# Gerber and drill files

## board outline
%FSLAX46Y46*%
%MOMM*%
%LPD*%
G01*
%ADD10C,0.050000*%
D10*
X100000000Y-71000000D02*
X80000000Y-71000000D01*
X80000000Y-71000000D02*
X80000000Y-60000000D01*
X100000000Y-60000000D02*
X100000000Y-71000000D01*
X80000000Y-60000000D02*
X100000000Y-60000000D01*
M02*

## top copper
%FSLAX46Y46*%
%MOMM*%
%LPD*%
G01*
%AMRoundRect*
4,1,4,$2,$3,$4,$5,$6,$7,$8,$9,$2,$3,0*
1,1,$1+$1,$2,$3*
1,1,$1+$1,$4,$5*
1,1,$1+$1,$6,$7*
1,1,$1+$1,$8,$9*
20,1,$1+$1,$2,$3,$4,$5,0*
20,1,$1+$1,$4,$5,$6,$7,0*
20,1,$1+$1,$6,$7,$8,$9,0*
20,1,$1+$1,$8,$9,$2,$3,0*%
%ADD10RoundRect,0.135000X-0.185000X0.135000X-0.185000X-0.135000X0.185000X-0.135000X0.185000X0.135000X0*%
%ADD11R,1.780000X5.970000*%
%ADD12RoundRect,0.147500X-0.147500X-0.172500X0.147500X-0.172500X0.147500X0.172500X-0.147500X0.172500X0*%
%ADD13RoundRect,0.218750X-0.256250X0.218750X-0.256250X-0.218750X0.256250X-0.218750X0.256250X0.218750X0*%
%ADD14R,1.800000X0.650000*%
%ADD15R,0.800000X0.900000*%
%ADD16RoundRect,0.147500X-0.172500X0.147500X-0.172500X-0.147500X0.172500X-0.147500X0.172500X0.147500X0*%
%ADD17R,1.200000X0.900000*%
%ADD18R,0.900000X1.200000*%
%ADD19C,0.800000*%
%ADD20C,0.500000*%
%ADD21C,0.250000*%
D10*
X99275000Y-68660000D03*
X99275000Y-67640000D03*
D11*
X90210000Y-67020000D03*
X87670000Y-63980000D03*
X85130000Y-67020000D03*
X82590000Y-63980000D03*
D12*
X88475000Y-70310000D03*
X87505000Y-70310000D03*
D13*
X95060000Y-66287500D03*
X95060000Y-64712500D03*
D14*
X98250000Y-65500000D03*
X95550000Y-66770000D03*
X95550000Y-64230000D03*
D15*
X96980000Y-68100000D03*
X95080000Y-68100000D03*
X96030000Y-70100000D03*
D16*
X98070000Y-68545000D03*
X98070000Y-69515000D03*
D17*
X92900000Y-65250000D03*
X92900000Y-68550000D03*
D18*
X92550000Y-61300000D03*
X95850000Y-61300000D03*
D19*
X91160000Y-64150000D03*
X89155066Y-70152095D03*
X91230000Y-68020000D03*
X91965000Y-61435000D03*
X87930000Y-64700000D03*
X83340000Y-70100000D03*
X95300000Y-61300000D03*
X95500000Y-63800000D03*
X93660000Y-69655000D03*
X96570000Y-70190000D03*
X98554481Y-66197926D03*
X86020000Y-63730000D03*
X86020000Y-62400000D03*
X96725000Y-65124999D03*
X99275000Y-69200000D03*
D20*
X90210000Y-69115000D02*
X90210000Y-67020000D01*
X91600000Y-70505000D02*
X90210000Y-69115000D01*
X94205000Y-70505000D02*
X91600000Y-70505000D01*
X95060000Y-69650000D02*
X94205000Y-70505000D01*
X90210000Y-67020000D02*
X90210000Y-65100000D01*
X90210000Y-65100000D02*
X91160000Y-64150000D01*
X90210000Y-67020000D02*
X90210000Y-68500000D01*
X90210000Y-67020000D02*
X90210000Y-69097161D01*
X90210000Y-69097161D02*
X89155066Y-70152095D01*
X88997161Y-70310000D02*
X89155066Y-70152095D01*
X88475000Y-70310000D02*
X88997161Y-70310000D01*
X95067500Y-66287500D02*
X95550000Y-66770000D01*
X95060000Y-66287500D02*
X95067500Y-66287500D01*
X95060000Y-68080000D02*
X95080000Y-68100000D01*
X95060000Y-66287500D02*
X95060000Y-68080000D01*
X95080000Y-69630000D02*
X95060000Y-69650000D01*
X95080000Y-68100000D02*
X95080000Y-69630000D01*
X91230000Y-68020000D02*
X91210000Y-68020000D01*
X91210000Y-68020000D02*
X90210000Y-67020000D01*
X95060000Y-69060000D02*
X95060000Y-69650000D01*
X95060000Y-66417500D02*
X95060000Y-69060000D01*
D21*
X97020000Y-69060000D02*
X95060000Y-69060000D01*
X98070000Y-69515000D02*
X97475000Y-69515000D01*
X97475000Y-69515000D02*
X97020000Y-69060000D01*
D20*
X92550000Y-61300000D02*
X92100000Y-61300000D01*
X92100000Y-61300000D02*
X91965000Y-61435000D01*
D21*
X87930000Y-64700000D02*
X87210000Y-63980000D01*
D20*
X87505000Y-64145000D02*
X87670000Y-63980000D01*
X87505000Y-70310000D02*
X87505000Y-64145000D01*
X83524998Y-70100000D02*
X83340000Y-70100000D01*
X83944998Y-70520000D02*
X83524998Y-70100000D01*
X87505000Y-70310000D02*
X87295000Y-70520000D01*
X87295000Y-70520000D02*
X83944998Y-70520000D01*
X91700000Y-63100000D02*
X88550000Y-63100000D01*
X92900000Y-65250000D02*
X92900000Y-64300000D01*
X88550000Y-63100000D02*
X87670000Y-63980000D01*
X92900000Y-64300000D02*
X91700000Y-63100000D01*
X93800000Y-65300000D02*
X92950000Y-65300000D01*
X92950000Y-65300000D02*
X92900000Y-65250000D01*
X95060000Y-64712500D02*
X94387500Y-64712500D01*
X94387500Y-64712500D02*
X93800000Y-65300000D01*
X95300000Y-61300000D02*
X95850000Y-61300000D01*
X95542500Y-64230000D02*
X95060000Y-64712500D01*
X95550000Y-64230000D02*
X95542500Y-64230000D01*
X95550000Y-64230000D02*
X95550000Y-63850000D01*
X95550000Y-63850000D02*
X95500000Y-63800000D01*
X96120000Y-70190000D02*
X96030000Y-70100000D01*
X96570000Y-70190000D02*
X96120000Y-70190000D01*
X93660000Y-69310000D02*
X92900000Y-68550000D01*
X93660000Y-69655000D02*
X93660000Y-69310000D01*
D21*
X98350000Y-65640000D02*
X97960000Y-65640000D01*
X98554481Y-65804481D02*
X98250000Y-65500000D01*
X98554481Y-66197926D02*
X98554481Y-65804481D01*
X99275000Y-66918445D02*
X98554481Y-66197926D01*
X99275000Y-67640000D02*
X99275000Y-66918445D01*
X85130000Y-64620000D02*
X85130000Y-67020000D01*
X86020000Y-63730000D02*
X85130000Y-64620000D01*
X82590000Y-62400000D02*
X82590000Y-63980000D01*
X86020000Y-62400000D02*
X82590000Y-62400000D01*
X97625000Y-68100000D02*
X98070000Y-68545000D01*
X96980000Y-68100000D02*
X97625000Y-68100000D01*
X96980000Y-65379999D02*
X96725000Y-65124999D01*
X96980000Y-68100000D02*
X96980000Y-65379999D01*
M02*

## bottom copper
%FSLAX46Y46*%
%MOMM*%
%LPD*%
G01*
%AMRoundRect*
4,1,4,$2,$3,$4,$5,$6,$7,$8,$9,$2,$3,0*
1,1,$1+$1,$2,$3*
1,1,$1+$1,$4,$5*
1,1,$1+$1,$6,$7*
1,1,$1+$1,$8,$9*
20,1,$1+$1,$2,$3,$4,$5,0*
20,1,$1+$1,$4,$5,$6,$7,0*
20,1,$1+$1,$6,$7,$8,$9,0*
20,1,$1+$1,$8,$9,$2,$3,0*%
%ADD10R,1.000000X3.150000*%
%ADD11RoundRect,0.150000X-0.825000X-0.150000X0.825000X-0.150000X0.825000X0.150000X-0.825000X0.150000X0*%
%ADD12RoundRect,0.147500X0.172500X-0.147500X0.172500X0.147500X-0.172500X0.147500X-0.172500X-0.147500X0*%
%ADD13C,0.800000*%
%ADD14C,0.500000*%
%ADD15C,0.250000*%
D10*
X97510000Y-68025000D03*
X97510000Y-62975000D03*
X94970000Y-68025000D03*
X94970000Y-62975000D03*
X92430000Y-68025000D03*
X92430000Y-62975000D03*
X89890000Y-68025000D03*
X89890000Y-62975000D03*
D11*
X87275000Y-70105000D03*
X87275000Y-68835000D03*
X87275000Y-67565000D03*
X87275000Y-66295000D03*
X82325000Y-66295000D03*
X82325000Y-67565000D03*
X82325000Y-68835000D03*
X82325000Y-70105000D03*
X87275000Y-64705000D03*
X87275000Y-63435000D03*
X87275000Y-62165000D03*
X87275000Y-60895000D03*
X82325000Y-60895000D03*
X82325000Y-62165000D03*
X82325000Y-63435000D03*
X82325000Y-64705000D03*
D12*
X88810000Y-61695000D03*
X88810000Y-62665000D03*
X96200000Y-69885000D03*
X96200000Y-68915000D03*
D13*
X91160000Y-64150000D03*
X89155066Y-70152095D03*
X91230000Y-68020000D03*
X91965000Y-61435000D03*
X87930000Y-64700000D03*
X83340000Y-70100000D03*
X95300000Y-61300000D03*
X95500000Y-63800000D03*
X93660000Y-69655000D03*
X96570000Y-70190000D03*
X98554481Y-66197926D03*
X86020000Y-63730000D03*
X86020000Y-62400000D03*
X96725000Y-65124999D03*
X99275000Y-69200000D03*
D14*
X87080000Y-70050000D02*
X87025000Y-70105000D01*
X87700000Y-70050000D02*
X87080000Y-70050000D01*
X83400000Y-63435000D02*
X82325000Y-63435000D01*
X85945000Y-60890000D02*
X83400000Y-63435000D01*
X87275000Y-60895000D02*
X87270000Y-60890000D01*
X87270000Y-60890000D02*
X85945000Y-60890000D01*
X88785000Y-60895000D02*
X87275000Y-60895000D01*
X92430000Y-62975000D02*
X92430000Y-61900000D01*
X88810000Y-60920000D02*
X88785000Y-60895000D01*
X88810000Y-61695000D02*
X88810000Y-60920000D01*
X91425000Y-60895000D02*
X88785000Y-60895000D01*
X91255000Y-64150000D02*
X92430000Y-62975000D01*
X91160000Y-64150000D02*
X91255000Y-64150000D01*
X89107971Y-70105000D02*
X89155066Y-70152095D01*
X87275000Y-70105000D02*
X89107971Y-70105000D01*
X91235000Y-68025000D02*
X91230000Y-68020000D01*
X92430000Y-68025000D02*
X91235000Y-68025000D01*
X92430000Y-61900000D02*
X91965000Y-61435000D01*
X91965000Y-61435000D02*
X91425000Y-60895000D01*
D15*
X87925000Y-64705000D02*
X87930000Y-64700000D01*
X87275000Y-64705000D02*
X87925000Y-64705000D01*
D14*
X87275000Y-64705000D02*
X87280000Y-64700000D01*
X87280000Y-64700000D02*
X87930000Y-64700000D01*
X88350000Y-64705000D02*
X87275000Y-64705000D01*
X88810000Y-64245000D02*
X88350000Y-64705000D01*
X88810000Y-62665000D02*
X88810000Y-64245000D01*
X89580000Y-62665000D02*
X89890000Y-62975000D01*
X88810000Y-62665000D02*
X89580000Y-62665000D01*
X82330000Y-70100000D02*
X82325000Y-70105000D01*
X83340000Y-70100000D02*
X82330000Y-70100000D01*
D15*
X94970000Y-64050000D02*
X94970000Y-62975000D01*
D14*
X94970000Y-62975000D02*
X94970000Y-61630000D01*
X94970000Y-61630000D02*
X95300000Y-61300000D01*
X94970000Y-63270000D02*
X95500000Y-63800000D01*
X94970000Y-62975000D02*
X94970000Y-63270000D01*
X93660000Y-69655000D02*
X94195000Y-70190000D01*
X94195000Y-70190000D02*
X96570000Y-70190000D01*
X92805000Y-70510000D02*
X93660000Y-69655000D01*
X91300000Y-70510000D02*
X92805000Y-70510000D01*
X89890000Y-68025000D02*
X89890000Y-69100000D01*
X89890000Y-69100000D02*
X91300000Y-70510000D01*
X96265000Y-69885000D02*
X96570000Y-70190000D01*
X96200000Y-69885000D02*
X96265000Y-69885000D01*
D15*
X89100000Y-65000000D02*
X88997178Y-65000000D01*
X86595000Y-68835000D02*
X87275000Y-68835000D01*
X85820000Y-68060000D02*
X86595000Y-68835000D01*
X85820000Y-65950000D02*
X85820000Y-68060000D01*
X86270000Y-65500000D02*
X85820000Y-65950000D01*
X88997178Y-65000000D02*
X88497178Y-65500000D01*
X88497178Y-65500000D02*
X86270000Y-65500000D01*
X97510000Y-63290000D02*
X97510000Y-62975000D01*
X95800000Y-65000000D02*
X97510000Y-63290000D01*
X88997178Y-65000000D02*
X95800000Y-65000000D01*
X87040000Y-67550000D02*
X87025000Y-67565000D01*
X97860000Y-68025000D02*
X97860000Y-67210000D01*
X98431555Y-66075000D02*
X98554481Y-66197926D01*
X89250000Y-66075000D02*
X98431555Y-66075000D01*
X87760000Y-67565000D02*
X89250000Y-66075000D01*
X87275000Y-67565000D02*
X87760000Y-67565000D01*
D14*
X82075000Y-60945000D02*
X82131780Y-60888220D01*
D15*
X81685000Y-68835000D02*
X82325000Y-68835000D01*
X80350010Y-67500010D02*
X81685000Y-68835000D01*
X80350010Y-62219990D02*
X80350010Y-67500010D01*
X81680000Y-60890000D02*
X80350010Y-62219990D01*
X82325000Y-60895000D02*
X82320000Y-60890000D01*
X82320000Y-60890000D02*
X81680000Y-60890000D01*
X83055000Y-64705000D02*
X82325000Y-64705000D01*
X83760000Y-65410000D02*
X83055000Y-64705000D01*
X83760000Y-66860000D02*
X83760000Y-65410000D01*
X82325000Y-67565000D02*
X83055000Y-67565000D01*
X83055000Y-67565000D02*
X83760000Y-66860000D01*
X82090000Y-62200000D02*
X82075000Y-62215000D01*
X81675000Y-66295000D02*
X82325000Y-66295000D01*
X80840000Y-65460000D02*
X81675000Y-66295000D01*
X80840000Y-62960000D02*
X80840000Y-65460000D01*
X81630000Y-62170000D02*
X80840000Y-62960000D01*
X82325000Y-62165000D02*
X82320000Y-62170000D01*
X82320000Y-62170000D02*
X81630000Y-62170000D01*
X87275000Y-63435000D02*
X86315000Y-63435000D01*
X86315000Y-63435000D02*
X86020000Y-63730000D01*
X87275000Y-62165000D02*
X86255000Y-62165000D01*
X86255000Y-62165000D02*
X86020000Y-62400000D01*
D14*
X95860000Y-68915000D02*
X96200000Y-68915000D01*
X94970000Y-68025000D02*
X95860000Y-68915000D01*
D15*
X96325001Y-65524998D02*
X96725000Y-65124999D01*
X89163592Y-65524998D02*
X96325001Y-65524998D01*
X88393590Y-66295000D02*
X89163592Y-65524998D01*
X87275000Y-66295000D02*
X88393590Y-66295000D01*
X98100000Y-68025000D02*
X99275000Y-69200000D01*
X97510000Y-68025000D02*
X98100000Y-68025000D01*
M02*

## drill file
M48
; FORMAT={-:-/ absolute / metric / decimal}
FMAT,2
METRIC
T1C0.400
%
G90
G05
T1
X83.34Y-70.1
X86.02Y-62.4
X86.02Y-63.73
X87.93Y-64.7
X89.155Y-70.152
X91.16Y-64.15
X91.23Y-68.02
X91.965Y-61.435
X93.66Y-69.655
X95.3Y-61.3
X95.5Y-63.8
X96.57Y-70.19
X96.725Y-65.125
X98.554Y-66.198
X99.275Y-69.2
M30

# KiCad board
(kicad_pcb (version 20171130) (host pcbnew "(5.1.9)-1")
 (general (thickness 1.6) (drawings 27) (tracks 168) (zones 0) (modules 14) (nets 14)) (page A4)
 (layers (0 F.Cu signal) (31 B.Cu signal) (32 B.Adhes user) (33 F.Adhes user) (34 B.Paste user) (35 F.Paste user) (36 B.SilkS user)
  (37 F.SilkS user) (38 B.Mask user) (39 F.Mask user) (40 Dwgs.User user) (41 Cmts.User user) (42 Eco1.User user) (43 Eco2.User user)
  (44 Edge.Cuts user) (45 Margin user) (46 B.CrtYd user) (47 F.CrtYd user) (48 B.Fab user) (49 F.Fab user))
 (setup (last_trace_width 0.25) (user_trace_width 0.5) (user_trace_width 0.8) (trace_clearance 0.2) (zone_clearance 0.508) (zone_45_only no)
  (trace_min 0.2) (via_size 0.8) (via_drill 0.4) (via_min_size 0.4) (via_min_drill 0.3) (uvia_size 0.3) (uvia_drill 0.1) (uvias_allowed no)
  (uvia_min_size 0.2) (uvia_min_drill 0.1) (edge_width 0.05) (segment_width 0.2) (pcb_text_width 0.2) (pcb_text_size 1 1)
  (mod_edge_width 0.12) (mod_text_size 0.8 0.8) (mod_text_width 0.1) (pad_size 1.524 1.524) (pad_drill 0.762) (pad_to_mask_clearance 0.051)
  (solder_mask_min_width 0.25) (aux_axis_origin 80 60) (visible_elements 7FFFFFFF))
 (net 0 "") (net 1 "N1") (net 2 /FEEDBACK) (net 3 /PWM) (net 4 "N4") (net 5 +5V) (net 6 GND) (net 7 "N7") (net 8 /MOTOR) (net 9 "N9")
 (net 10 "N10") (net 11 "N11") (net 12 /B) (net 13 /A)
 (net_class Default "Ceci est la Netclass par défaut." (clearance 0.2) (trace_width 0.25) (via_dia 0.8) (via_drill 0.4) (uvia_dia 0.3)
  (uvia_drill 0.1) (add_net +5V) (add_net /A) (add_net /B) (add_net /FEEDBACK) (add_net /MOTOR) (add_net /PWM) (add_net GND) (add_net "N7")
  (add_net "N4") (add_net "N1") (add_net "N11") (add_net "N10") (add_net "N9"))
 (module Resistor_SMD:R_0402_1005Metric (layer F.Cu) (at 99.275 68.15 270)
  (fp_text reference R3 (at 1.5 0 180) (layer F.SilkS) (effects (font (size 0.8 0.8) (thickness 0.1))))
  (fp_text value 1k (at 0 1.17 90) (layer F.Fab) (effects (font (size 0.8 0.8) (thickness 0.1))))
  (pad 2 smd roundrect (at 0.51 0 270) (size 0.54 0.64) (layers F.Cu F.Paste F.Mask) (roundrect_rratio 0.25) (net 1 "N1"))
  (pad 1 smd roundrect (at -0.51 0 270) (size 0.54 0.64) (layers F.Cu F.Paste F.Mask) (roundrect_rratio 0.25) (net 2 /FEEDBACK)))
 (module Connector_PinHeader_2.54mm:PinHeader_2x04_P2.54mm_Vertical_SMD (layer B.Cu) (at 93.7 65.5 270)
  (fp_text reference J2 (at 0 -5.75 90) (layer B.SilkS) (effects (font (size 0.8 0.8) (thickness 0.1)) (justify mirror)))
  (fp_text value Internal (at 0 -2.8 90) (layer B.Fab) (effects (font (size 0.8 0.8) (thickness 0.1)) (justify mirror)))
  (pad 8 smd rect (at 2.525 -3.81 270) (size 3.15 1) (layers B.Cu B.Paste B.Mask) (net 1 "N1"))
  (pad 7 smd rect (at -2.525 -3.81 270) (size 3.15 1) (layers B.Cu B.Paste B.Mask) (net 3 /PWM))
  (pad 6 smd rect (at 2.525 -1.27 270) (size 3.15 1) (layers B.Cu B.Paste B.Mask) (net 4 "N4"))
  (pad 5 smd rect (at -2.525 -1.27 270) (size 3.15 1) (layers B.Cu B.Paste B.Mask) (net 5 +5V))
  (pad 4 smd rect (at 2.525 1.27 270) (size 3.15 1) (layers B.Cu B.Paste B.Mask) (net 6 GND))
  (pad 3 smd rect (at -2.525 1.27 270) (size 3.15 1) (layers B.Cu B.Paste B.Mask) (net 6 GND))
  (pad 2 smd rect (at 2.525 3.81 270) (size 3.15 1) (layers B.Cu B.Paste B.Mask) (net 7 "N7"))
  (pad 1 smd rect (at -2.525 3.81 270) (size 3.15 1) (layers B.Cu B.Paste B.Mask) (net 5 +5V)))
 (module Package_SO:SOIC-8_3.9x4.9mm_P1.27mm (layer B.Cu) (at 84.8 68.2)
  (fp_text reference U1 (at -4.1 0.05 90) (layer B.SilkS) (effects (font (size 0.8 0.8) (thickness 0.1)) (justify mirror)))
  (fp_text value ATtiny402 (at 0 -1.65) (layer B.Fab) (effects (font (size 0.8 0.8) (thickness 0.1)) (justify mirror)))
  (pad 8 smd roundrect (at 2.475 1.905) (size 1.95 0.6) (layers B.Cu B.Paste B.Mask) (roundrect_rratio 0.25) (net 6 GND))
  (pad 7 smd roundrect (at 2.475 0.635) (size 1.95 0.6) (layers B.Cu B.Paste B.Mask) (roundrect_rratio 0.25) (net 3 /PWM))
  (pad 6 smd roundrect (at 2.475 -0.635) (size 1.95 0.6) (layers B.Cu B.Paste B.Mask) (roundrect_rratio 0.25) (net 2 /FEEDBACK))
  (pad 5 smd roundrect (at 2.475 -1.905) (size 1.95 0.6) (layers B.Cu B.Paste B.Mask) (roundrect_rratio 0.25) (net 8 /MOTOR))
  (pad 4 smd roundrect (at -2.475 -1.905) (size 1.95 0.6) (layers B.Cu B.Paste B.Mask) (roundrect_rratio 0.25) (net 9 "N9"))
  (pad 3 smd roundrect (at -2.475 -0.635) (size 1.95 0.6) (layers B.Cu B.Paste B.Mask) (roundrect_rratio 0.25) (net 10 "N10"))
  (pad 2 smd roundrect (at -2.475 0.635) (size 1.95 0.6) (layers B.Cu B.Paste B.Mask) (roundrect_rratio 0.25) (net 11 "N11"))
  (pad 1 smd roundrect (at -2.475 1.905) (size 1.95 0.6) (layers B.Cu B.Paste B.Mask) (roundrect_rratio 0.25) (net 5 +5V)))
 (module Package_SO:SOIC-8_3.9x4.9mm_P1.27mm (layer B.Cu) (at 84.8 62.8)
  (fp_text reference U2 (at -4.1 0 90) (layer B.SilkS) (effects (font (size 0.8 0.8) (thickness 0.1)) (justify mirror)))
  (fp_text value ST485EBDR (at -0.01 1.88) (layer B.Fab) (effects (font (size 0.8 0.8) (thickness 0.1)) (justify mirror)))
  (pad 8 smd roundrect (at 2.475 1.905) (size 1.95 0.6) (layers B.Cu B.Paste B.Mask) (roundrect_rratio 0.25) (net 5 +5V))
  (pad 7 smd roundrect (at 2.475 0.635) (size 1.95 0.6) (layers B.Cu B.Paste B.Mask) (roundrect_rratio 0.25) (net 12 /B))
  (pad 6 smd roundrect (at 2.475 -0.635) (size 1.95 0.6) (layers B.Cu B.Paste B.Mask) (roundrect_rratio 0.25) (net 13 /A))
  (pad 5 smd roundrect (at 2.475 -1.905) (size 1.95 0.6) (layers B.Cu B.Paste B.Mask) (roundrect_rratio 0.25) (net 6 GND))
  (pad 4 smd roundrect (at -2.475 -1.905) (size 1.95 0.6) (layers B.Cu B.Paste B.Mask) (roundrect_rratio 0.25) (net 11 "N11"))
  (pad 3 smd roundrect (at -2.475 -0.635) (size 1.95 0.6) (layers B.Cu B.Paste B.Mask) (roundrect_rratio 0.25) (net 9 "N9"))
  (pad 2 smd roundrect (at -2.475 0.635) (size 1.95 0.6) (layers B.Cu B.Paste B.Mask) (roundrect_rratio 0.25) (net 6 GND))
  (pad 1 smd roundrect (at -2.475 1.905) (size 1.95 0.6) (layers B.Cu B.Paste B.Mask) (roundrect_rratio 0.25) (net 10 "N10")))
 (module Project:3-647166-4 (layer F.Cu) (at 86.4 65.5 180)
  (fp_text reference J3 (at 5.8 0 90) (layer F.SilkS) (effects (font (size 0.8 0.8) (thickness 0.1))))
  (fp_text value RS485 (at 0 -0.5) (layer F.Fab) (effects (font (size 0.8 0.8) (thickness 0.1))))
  (pad 4 smd rect (at -3.81 -1.52 180) (size 1.78 5.97) (layers F.Cu F.Paste F.Mask) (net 6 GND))
  (pad 3 smd rect (at -1.27 1.52 180) (size 1.78 5.97) (layers F.Cu F.Paste F.Mask) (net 5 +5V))
  (pad 2 smd rect (at 1.27 -1.52 180) (size 1.78 5.97) (layers F.Cu F.Paste F.Mask) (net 12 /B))
  (pad 1 smd rect (at 3.81 1.52 180) (size 1.78 5.97) (layers F.Cu F.Paste F.Mask) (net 13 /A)))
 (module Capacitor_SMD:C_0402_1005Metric (layer F.Cu) (at 87.99 70.31)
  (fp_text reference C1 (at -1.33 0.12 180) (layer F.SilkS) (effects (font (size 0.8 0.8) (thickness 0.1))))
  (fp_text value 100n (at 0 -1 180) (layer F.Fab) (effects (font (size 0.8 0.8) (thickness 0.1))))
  (pad 2 smd roundrect (at 0.485 0) (size 0.59 0.64) (layers F.Cu F.Paste F.Mask) (roundrect_rratio 0.25) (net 6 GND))
  (pad 1 smd roundrect (at -0.485 0) (size 0.59 0.64) (layers F.Cu F.Paste F.Mask) (roundrect_rratio 0.25) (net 5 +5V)))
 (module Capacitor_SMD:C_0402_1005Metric (layer B.Cu) (at 88.81 62.18 90)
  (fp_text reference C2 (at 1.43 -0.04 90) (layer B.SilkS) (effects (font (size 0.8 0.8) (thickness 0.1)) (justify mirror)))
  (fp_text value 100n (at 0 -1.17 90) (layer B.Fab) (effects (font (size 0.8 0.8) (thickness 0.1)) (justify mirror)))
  (pad 2 smd roundrect (at 0.485 0 90) (size 0.59 0.64) (layers B.Cu B.Paste B.Mask) (roundrect_rratio 0.25) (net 6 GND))
  (pad 1 smd roundrect (at -0.485 0 90) (size 0.59 0.64) (layers B.Cu B.Paste B.Mask) (roundrect_rratio 0.25) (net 5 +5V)))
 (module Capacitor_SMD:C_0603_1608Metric (layer F.Cu) (at 95.06 65.5 270)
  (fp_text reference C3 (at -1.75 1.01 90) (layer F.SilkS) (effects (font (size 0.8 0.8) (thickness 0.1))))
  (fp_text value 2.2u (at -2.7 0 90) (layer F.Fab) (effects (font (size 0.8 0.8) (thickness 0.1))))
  (pad 2 smd roundrect (at 0.7875 0 270) (size 0.875 0.95) (layers F.Cu F.Paste F.Mask) (roundrect_rratio 0.25) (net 6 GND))
  (pad 1 smd roundrect (at -0.7875 0 270) (size 0.875 0.95) (layers F.Cu F.Paste F.Mask) (roundrect_rratio 0.25) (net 5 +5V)))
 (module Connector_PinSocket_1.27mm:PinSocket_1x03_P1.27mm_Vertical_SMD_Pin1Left (layer F.Cu) (at 96.9 65.5)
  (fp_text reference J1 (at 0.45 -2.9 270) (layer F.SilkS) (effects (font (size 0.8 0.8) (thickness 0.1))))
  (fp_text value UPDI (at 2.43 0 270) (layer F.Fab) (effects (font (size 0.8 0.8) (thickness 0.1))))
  (pad 2 smd rect (at 1.35 0) (size 1.8 0.65) (layers F.Cu F.Paste F.Mask) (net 2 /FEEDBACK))
  (pad 3 smd rect (at -1.35 1.27) (size 1.8 0.65) (layers F.Cu F.Paste F.Mask) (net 6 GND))
  (pad 1 smd rect (at -1.35 -1.27) (size 1.8 0.65) (layers F.Cu F.Paste F.Mask) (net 5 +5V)))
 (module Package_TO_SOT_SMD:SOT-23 (layer F.Cu) (at 96.03 69.1 270)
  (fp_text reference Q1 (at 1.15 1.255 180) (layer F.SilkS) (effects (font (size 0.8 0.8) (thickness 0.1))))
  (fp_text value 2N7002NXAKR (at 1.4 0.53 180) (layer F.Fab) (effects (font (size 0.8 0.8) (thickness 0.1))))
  (pad 1 smd rect (at -1 -0.95 270) (size 0.9 0.8) (layers F.Cu F.Paste F.Mask) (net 8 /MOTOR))
  (pad 2 smd rect (at -1 0.95 270) (size 0.9 0.8) (layers F.Cu F.Paste F.Mask) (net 6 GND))
  (pad 3 smd rect (at 1 0 270) (size 0.9 0.8) (layers F.Cu F.Paste F.Mask) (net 7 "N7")))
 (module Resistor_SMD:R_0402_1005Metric (layer F.Cu) (at 98.07 69.03 270)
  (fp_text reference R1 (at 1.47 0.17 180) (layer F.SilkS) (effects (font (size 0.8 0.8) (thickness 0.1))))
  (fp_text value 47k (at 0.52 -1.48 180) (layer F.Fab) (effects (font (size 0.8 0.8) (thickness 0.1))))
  (pad 1 smd roundrect (at -0.485 0 270) (size 0.59 0.64) (layers F.Cu F.Paste F.Mask) (roundrect_rratio 0.25) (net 8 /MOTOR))
  (pad 2 smd roundrect (at 0.485 0 270) (size 0.59 0.64) (layers F.Cu F.Paste F.Mask) (roundrect_rratio 0.25) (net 6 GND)))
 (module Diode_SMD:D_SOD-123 (layer F.Cu) (at 92.9 66.9 270)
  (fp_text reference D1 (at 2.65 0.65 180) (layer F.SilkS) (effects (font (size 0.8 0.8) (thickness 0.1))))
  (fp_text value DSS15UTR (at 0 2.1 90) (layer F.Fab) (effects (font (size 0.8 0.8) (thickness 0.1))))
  (pad 1 smd rect (at -1.65 0 270) (size 0.9 1.2) (layers F.Cu F.Paste F.Mask) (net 5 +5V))
  (pad 2 smd rect (at 1.65 0 270) (size 0.9 1.2) (layers F.Cu F.Paste F.Mask) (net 7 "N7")))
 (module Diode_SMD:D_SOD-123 (layer F.Cu) (at 94.2 61.3 180)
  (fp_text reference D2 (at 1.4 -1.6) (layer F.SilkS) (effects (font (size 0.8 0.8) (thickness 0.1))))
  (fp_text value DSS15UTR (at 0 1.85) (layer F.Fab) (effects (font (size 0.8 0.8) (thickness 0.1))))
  (pad 2 smd rect (at 1.65 0 180) (size 0.9 1.2) (layers F.Cu F.Paste F.Mask) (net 6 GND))
  (pad 1 smd rect (at -1.65 0 180) (size 0.9 1.2) (layers F.Cu F.Paste F.Mask) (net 5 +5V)))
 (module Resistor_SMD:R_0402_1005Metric (layer B.Cu) (at 96.2 69.4 90)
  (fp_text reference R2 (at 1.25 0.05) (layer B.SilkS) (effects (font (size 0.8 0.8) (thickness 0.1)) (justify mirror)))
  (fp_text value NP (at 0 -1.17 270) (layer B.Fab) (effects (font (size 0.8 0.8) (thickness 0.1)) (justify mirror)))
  (pad 1 smd roundrect (at -0.485 0 90) (size 0.59 0.64) (layers B.Cu B.Paste B.Mask) (roundrect_rratio 0.25) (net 7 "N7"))
  (pad 2 smd roundrect (at 0.485 0 90) (size 0.59 0.64) (layers B.Cu B.Paste B.Mask) (roundrect_rratio 0.25) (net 4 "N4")))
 (gr_line (start 100 71) (end 80 71) (layer Edge.Cuts) (width 0.05))
 (gr_line (start 80 71) (end 80 60) (layer Edge.Cuts) (width 0.05))
 (gr_line (start 100 60) (end 100 71) (layer Edge.Cuts) (width 0.05))
 (gr_line (start 80 60) (end 100 60) (layer Edge.Cuts) (width 0.05))
 (segment (start 87.08 70.05) (end 87.025 70.105) (width 0.5) (layer B.Cu) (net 6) (status 30))
 (segment (start 87.7 70.05) (end 87.08 70.05) (width 0.5) (layer B.Cu) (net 6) (status 30))
 (segment (start 83.4 63.435) (end 82.325 63.435) (width 0.5) (layer B.Cu) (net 6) (status 20))
 (segment (start 85.945 60.89) (end 83.4 63.435) (width 0.5) (layer B.Cu) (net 6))
 (segment (start 87.275 60.895) (end 87.27 60.89) (width 0.5) (layer B.Cu) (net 6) (status 30))
 (segment (start 87.27 60.89) (end 85.945 60.89) (width 0.5) (layer B.Cu) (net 6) (status 10))
 (segment (start 90.21 69.115) (end 90.21 67.02) (width 0.5) (layer F.Cu) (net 6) (status 30))
 (segment (start 91.6 70.505) (end 90.21 69.115) (width 0.5) (layer F.Cu) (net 6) (status 20))
 (segment (start 94.205 70.505) (end 91.6 70.505) (width 0.5) (layer F.Cu) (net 6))
 (segment (start 95.06 69.65) (end 94.205 70.505) (width 0.5) (layer F.Cu) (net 6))
 (segment (start 88.785 60.895) (end 87.275 60.895) (width 0.5) (layer B.Cu) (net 6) (status 20))
 (segment (start 92.43 62.975) (end 92.43 61.9) (width 0.5) (layer B.Cu) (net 6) (status 30))
 (segment (start 88.81 60.92) (end 88.785 60.895) (width 0.5) (layer B.Cu) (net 6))
 (segment (start 88.81 61.695) (end 88.81 60.92) (width 0.5) (layer B.Cu) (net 6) (status 10))
 (segment (start 91.425 60.895) (end 88.785 60.895) (width 0.5) (layer B.Cu) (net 6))
 (via (at 91.16 64.15) (size 0.8) (drill 0.4) (layers F.Cu B.Cu) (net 6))
 (segment (start 90.21 67.02) (end 90.21 65.1) (width 0.5) (layer F.Cu) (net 6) (status 30))
 (segment (start 90.21 65.1) (end 91.16 64.15) (width 0.5) (layer F.Cu) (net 6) (status 10))
 (segment (start 91.255 64.15) (end 92.43 62.975) (width 0.5) (layer B.Cu) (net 6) (status 20))
 (segment (start 91.16 64.15) (end 91.255 64.15) (width 0.5) (layer B.Cu) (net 6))
 (segment (start 90.21 67.02) (end 90.21 68.5) (width 0.5) (layer F.Cu) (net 6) (status 30))
 (via (at 89.155066 70.152095) (size 0.8) (drill 0.4) (layers F.Cu B.Cu) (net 6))
 (segment (start 90.21 67.02) (end 90.21 69.097161) (width 0.5) (layer F.Cu) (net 6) (status 30))
 (segment (start 90.21 69.097161) (end 89.155066 70.152095) (width 0.5) (layer F.Cu) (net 6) (status 10))
 (segment (start 89.107971 70.105) (end 89.155066 70.152095) (width 0.5) (layer B.Cu) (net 6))
 (segment (start 87.275 70.105) (end 89.107971 70.105) (width 0.5) (layer B.Cu) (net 6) (status 10))
 (segment (start 88.997161 70.31) (end 89.155066 70.152095) (width 0.5) (layer F.Cu) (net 6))
 (segment (start 88.475 70.31) (end 88.997161 70.31) (width 0.5) (layer F.Cu) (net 6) (status 10))
 (segment (start 95.0675 66.2875) (end 95.55 66.77) (width 0.5) (layer F.Cu) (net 6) (status 30))
 (segment (start 95.06 66.2875) (end 95.0675 66.2875) (width 0.5) (layer F.Cu) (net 6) (status 30))
 (segment (start 95.06 68.08) (end 95.08 68.1) (width 0.5) (layer F.Cu) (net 6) (status 30))
 (segment (start 95.06 66.2875) (end 95.06 68.08) (width 0.5) (layer F.Cu) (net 6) (status 30))
 (segment (start 95.08 69.63) (end 95.06 69.65) (width 0.5) (layer F.Cu) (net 6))
 (segment (start 95.08 68.1) (end 95.08 69.63) (width 0.5) (layer F.Cu) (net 6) (status 10))
 (segment (start 91.23 68.02) (end 91.21 68.02) (width 0.5) (layer F.Cu) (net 6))
 (segment (start 91.21 68.02) (end 90.21 67.02) (width 0.5) (layer F.Cu) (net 6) (status 20))
 (segment (start 91.235 68.025) (end 91.23 68.02) (width 0.5) (layer B.Cu) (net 6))
 (via (at 91.23 68.02) (size 0.8) (drill 0.4) (layers F.Cu B.Cu) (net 6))
 (segment (start 92.43 68.025) (end 91.235 68.025) (width 0.5) (layer B.Cu) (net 6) (status 10))
 (segment (start 95.06 69.06) (end 95.06 69.65) (width 0.5) (layer F.Cu) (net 6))
 (segment (start 95.06 66.4175) (end 95.06 69.06) (width 0.5) (layer F.Cu) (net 6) (status 10))
 (segment (start 97.02 69.06) (end 95.06 69.06) (width 0.25) (layer F.Cu) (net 6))
 (segment (start 98.07 69.515) (end 97.475 69.515) (width 0.25) (layer F.Cu) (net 6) (status 10))
 (segment (start 97.475 69.515) (end 97.02 69.06) (width 0.25) (layer F.Cu) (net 6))
 (via (at 91.965 61.435) (size 0.8) (drill 0.4) (layers F.Cu B.Cu) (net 6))
 (segment (start 92.55 61.3) (end 92.1 61.3) (width 0.5) (layer F.Cu) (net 6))
 (segment (start 92.1 61.3) (end 91.965 61.435) (width 0.5) (layer F.Cu) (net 6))
 (segment (start 92.43 61.9) (end 91.965 61.435) (width 0.5) (layer B.Cu) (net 6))
 (segment (start 91.965 61.435) (end 91.425 60.895) (width 0.5) (layer B.Cu) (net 6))
 (via (at 87.93 64.7) (size 0.8) (drill 0.4) (layers F.Cu B.Cu) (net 5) (status 30))
 (segment (start 87.925 64.705) (end 87.93 64.7) (width 0.25) (layer B.Cu) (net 5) (status 30))
 (segment (start 87.275 64.705) (end 87.925 64.705) (width 0.25) (layer B.Cu) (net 5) (status 30))
 (segment (start 87.93 64.7) (end 87.21 63.98) (width 0.25) (layer F.Cu) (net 5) (status 30))
 (segment (start 87.275 64.705) (end 87.28 64.7) (width 0.5) (layer B.Cu) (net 5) (status 30))
 (segment (start 87.28 64.7) (end 87.93 64.7) (width 0.5) (layer B.Cu) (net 5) (status 30))
 (segment (start 88.35 64.705) (end 87.275 64.705) (width 0.5) (layer B.Cu) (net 5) (status 20))
 (segment (start 88.81 64.245) (end 88.35 64.705) (width 0.5) (layer B.Cu) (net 5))
 (segment (start 88.81 62.665) (end 88.81 64.245) (width 0.5) (layer B.Cu) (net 5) (status 10))
 (segment (start 89.58 62.665) (end 89.89 62.975) (width 0.5) (layer B.Cu) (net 5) (status 30))
 (segment (start 88.81 62.665) (end 89.58 62.665) (width 0.5) (layer B.Cu) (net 5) (status 30))
 (via (at 83.34 70.1) (size 0.8) (drill 0.4) (layers F.Cu B.Cu) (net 5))
 (segment (start 82.33 70.1) (end 82.325 70.105) (width 0.5) (layer B.Cu) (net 5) (status 30))
 (segment (start 83.34 70.1) (end 82.33 70.1) (width 0.5) (layer B.Cu) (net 5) (status 20))
 (segment (start 87.505 64.145) (end 87.67 63.98) (width 0.5) (layer F.Cu) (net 5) (status 30))
 (segment (start 87.505 70.31) (end 87.505 64.145) (width 0.5) (layer F.Cu) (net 5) (status 30))
 (segment (start 83.524998 70.1) (end 83.34 70.1) (width 0.5) (layer F.Cu) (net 5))
 (segment (start 83.944998 70.52) (end 83.524998 70.1) (width 0.5) (layer F.Cu) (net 5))
 (segment (start 87.505 70.31) (end 87.295 70.52) (width 0.5) (layer F.Cu) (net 5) (status 30))
 (segment (start 87.295 70.52) (end 83.944998 70.52) (width 0.5) (layer F.Cu) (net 5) (status 10))
 (segment (start 91.7 63.1) (end 88.55 63.1) (width 0.5) (layer F.Cu) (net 5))
 (segment (start 92.9 65.25) (end 92.9 64.3) (width 0.5) (layer F.Cu) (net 5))
 (segment (start 88.55 63.1) (end 87.67 63.98) (width 0.5) (layer F.Cu) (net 5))
 (segment (start 92.9 64.3) (end 91.7 63.1) (width 0.5) (layer F.Cu) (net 5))
 (segment (start 93.8 65.3) (end 92.95 65.3) (width 0.5) (layer F.Cu) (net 5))
 (segment (start 92.95 65.3) (end 92.9 65.25) (width 0.5) (layer F.Cu) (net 5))
 (segment (start 95.06 64.7125) (end 94.3875 64.7125) (width 0.5) (layer F.Cu) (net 5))
 (segment (start 94.3875 64.7125) (end 93.8 65.3) (width 0.5) (layer F.Cu) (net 5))
 (segment (start 94.97 64.05) (end 94.97 62.975) (width 0.25) (layer B.Cu) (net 5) (status 30))
 (via (at 95.3 61.3) (size 0.8) (drill 0.4) (layers F.Cu B.Cu) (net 5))
 (segment (start 94.97 62.975) (end 94.97 61.63) (width 0.5) (layer B.Cu) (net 5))
 (segment (start 94.97 61.63) (end 95.3 61.3) (width 0.5) (layer B.Cu) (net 5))
 (segment (start 95.3 61.3) (end 95.85 61.3) (width 0.5) (layer F.Cu) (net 5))
 (segment (start 95.5425 64.23) (end 95.06 64.7125) (width 0.5) (layer F.Cu) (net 5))
 (segment (start 95.55 64.23) (end 95.5425 64.23) (width 0.5) (layer F.Cu) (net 5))
 (via (at 95.5 63.8) (size 0.8) (drill 0.4) (layers F.Cu B.Cu) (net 5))
 (segment (start 95.55 64.23) (end 95.55 63.85) (width 0.5) (layer F.Cu) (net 5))
 (segment (start 95.55 63.85) (end 95.5 63.8) (width 0.5) (layer F.Cu) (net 5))
 (segment (start 94.97 63.27) (end 95.5 63.8) (width 0.5) (layer B.Cu) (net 5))
 (segment (start 94.97 62.975) (end 94.97 63.27) (width 0.5) (layer B.Cu) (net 5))
 (via (at 93.66 69.655) (size 0.8) (drill 0.4) (layers F.Cu B.Cu) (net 7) (status 30))
 (via (at 96.57 70.19) (size 0.8) (drill 0.4) (layers F.Cu B.Cu) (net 7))
 (segment (start 93.66 69.655) (end 94.195 70.19) (width 0.5) (layer B.Cu) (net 7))
 (segment (start 94.195 70.19) (end 96.57 70.19) (width 0.5) (layer B.Cu) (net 7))
 (segment (start 96.12 70.19) (end 96.03 70.1) (width 0.5) (layer F.Cu) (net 7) (status 30))
 (segment (start 96.57 70.19) (end 96.12 70.19) (width 0.5) (layer F.Cu) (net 7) (status 20))
 (segment (start 92.805 70.51) (end 93.66 69.655) (width 0.5) (layer B.Cu) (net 7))
 (segment (start 91.3 70.51) (end 92.805 70.51) (width 0.5) (layer B.Cu) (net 7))
 (segment (start 89.89 68.025) (end 89.89 69.1) (width 0.5) (layer B.Cu) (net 7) (status 30))
 (segment (start 89.89 69.1) (end 91.3 70.51) (width 0.5) (layer B.Cu) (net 7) (status 10))
 (segment (start 93.66 69.31) (end 92.9 68.55) (width 0.5) (layer F.Cu) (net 7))
 (segment (start 93.66 69.655) (end 93.66 69.31) (width 0.5) (layer F.Cu) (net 7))
 (segment (start 96.265 69.885) (end 96.57 70.19) (width 0.5) (layer B.Cu) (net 7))
 (segment (start 96.2 69.885) (end 96.265 69.885) (width 0.5) (layer B.Cu) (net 7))
 (segment (start 89.1 65) (end 88.997178 65) (width 0.25) (layer B.Cu) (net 3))
 (segment (start 86.595 68.835) (end 87.275 68.835) (width 0.25) (layer B.Cu) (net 3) (status 30))
 (segment (start 85.82 68.06) (end 86.595 68.835) (width 0.25) (layer B.Cu) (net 3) (status 20))
 (segment (start 85.82 65.95) (end 85.82 68.06) (width 0.25) (layer B.Cu) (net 3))
 (segment (start 86.27 65.5) (end 85.82 65.95) (width 0.25) (layer B.Cu) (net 3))
 (segment (start 88.997178 65) (end 88.497178 65.5) (width 0.25) (layer B.Cu) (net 3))
 (segment (start 88.497178 65.5) (end 86.27 65.5) (width 0.25) (layer B.Cu) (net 3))
 (segment (start 97.51 63.29) (end 97.51 62.975) (width 0.25) (layer B.Cu) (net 3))
 (segment (start 95.8 65) (end 97.51 63.29) (width 0.25) (layer B.Cu) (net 3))
 (segment (start 88.997178 65) (end 95.8 65) (width 0.25) (layer B.Cu) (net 3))
 (segment (start 98.35 65.64) (end 97.96 65.64) (width 0.25) (layer F.Cu) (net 2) (status 30))
 (segment (start 87.04 67.55) (end 87.025 67.565) (width 0.25) (layer B.Cu) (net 2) (status 30))
 (segment (start 97.86 68.025) (end 97.86 67.21) (width 0.25) (layer B.Cu) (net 1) (status 30))
 (via (at 98.554481 66.197926) (size 0.8) (drill 0.4) (layers F.Cu B.Cu) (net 2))
 (segment (start 98.431555 66.075) (end 98.554481 66.197926) (width 0.25) (layer B.Cu) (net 2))
 (segment (start 89.25 66.075) (end 98.431555 66.075) (width 0.25) (layer B.Cu) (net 2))
 (segment (start 87.76 67.565) (end 89.25 66.075) (width 0.25) (layer B.Cu) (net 2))
 (segment (start 87.275 67.565) (end 87.76 67.565) (width 0.25) (layer B.Cu) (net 2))
 (segment (start 98.554481 65.804481) (end 98.25 65.5) (width 0.25) (layer F.Cu) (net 2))
 (segment (start 98.554481 66.197926) (end 98.554481 65.804481) (width 0.25) (layer F.Cu) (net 2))
 (segment (start 99.275 66.918445) (end 98.554481 66.197926) (width 0.25) (layer F.Cu) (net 2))
 (segment (start 99.275 67.64) (end 99.275 66.918445) (width 0.25) (layer F.Cu) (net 2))
 (segment (start 82.075 60.945) (end 82.13178 60.88822) (width 0.5) (layer B.Cu) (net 11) (status 30))
 (segment (start 81.685 68.835) (end 82.325 68.835) (width 0.25) (layer B.Cu) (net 11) (status 30))
 (segment (start 80.35001 67.50001) (end 81.685 68.835) (width 0.25) (layer B.Cu) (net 11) (status 20))
 (segment (start 80.35001 62.21999) (end 80.35001 67.50001) (width 0.25) (layer B.Cu) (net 11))
 (segment (start 81.68 60.89) (end 80.35001 62.21999) (width 0.25) (layer B.Cu) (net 11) (status 10))
 (segment (start 82.325 60.895) (end 82.32 60.89) (width 0.25) (layer B.Cu) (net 11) (status 30))
 (segment (start 82.32 60.89) (end 81.68 60.89) (width 0.25) (layer B.Cu) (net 11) (status 30))
 (segment (start 83.055 64.705) (end 82.325 64.705) (width 0.25) (layer B.Cu) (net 10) (status 30))
 (segment (start 83.76 65.41) (end 83.055 64.705) (width 0.25) (layer B.Cu) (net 10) (status 20))
 (segment (start 83.76 66.86) (end 83.76 65.41) (width 0.25) (layer B.Cu) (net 10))
 (segment (start 82.325 67.565) (end 83.055 67.565) (width 0.25) (layer B.Cu) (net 10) (status 30))
 (segment (start 83.055 67.565) (end 83.76 66.86) (width 0.25) (layer B.Cu) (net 10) (status 10))
 (segment (start 82.09 62.2) (end 82.075 62.215) (width 0.25) (layer B.Cu) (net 9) (status 30))
 (segment (start 81.675 66.295) (end 82.325 66.295) (width 0.25) (layer B.Cu) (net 9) (status 30))
 (segment (start 80.84 65.46) (end 81.675 66.295) (width 0.25) (layer B.Cu) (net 9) (status 20))
 (segment (start 80.84 62.96) (end 80.84 65.46) (width 0.25) (layer B.Cu) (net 9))
 (segment (start 81.63 62.17) (end 80.84 62.96) (width 0.25) (layer B.Cu) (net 9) (status 10))
 (segment (start 82.325 62.165) (end 82.32 62.17) (width 0.25) (layer B.Cu) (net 9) (status 30))
 (segment (start 82.32 62.17) (end 81.63 62.17) (width 0.25) (layer B.Cu) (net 9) (status 30))
 (via (at 86.02 63.73) (size 0.8) (drill 0.4) (layers F.Cu B.Cu) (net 12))
 (segment (start 87.275 63.435) (end 86.315 63.435) (width 0.25) (layer B.Cu) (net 12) (status 30))
 (segment (start 86.315 63.435) (end 86.02 63.73) (width 0.25) (layer B.Cu) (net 12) (status 10))
 (segment (start 85.13 64.62) (end 85.13 67.02) (width 0.25) (layer F.Cu) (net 12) (status 30))
 (segment (start 86.02 63.73) (end 85.13 64.62) (width 0.25) (layer F.Cu) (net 12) (status 20))
 (via (at 86.02 62.4) (size 0.8) (drill 0.4) (layers F.Cu B.Cu) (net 13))
 (segment (start 87.275 62.165) (end 86.255 62.165) (width 0.25) (layer B.Cu) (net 13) (status 10))
 (segment (start 86.255 62.165) (end 86.02 62.4) (width 0.25) (layer B.Cu) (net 13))
 (segment (start 82.59 62.4) (end 82.59 63.98) (width 0.25) (layer F.Cu) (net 13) (status 30))
 (segment (start 86.02 62.4) (end 82.59 62.4) (width 0.25) (layer F.Cu) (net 13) (status 20))
 (segment (start 95.86 68.915) (end 96.2 68.915) (width 0.5) (layer B.Cu) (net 4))
 (segment (start 94.97 68.025) (end 95.86 68.915) (width 0.5) (layer B.Cu) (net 4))
 (segment (start 97.625 68.1) (end 98.07 68.545) (width 0.25) (layer F.Cu) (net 8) (status 20))
 (segment (start 96.98 68.1) (end 97.625 68.1) (width 0.25) (layer F.Cu) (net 8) (status 10))
 (via (at 96.725 65.124999) (size 0.8) (drill 0.4) (layers F.Cu B.Cu) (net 8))
 (segment (start 96.98 65.379999) (end 96.725 65.124999) (width 0.25) (layer F.Cu) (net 8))
 (segment (start 96.98 68.1) (end 96.98 65.379999) (width 0.25) (layer F.Cu) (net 8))
 (segment (start 96.325001 65.524998) (end 96.725 65.124999) (width 0.25) (layer B.Cu) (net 8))
 (segment (start 89.163592 65.524998) (end 96.325001 65.524998) (width 0.25) (layer B.Cu) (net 8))
 (segment (start 88.39359 66.295) (end 89.163592 65.524998) (width 0.25) (layer B.Cu) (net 8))
 (segment (start 87.275 66.295) (end 88.39359 66.295) (width 0.25) (layer B.Cu) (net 8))
 (via (at 99.275 69.2) (size 0.8) (drill 0.4) (layers F.Cu B.Cu) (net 1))
 (segment (start 98.1 68.025) (end 99.275 69.2) (width 0.25) (layer B.Cu) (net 1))
 (segment (start 97.51 68.025) (end 98.1 68.025) (width 0.25) (layer B.Cu) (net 1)))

